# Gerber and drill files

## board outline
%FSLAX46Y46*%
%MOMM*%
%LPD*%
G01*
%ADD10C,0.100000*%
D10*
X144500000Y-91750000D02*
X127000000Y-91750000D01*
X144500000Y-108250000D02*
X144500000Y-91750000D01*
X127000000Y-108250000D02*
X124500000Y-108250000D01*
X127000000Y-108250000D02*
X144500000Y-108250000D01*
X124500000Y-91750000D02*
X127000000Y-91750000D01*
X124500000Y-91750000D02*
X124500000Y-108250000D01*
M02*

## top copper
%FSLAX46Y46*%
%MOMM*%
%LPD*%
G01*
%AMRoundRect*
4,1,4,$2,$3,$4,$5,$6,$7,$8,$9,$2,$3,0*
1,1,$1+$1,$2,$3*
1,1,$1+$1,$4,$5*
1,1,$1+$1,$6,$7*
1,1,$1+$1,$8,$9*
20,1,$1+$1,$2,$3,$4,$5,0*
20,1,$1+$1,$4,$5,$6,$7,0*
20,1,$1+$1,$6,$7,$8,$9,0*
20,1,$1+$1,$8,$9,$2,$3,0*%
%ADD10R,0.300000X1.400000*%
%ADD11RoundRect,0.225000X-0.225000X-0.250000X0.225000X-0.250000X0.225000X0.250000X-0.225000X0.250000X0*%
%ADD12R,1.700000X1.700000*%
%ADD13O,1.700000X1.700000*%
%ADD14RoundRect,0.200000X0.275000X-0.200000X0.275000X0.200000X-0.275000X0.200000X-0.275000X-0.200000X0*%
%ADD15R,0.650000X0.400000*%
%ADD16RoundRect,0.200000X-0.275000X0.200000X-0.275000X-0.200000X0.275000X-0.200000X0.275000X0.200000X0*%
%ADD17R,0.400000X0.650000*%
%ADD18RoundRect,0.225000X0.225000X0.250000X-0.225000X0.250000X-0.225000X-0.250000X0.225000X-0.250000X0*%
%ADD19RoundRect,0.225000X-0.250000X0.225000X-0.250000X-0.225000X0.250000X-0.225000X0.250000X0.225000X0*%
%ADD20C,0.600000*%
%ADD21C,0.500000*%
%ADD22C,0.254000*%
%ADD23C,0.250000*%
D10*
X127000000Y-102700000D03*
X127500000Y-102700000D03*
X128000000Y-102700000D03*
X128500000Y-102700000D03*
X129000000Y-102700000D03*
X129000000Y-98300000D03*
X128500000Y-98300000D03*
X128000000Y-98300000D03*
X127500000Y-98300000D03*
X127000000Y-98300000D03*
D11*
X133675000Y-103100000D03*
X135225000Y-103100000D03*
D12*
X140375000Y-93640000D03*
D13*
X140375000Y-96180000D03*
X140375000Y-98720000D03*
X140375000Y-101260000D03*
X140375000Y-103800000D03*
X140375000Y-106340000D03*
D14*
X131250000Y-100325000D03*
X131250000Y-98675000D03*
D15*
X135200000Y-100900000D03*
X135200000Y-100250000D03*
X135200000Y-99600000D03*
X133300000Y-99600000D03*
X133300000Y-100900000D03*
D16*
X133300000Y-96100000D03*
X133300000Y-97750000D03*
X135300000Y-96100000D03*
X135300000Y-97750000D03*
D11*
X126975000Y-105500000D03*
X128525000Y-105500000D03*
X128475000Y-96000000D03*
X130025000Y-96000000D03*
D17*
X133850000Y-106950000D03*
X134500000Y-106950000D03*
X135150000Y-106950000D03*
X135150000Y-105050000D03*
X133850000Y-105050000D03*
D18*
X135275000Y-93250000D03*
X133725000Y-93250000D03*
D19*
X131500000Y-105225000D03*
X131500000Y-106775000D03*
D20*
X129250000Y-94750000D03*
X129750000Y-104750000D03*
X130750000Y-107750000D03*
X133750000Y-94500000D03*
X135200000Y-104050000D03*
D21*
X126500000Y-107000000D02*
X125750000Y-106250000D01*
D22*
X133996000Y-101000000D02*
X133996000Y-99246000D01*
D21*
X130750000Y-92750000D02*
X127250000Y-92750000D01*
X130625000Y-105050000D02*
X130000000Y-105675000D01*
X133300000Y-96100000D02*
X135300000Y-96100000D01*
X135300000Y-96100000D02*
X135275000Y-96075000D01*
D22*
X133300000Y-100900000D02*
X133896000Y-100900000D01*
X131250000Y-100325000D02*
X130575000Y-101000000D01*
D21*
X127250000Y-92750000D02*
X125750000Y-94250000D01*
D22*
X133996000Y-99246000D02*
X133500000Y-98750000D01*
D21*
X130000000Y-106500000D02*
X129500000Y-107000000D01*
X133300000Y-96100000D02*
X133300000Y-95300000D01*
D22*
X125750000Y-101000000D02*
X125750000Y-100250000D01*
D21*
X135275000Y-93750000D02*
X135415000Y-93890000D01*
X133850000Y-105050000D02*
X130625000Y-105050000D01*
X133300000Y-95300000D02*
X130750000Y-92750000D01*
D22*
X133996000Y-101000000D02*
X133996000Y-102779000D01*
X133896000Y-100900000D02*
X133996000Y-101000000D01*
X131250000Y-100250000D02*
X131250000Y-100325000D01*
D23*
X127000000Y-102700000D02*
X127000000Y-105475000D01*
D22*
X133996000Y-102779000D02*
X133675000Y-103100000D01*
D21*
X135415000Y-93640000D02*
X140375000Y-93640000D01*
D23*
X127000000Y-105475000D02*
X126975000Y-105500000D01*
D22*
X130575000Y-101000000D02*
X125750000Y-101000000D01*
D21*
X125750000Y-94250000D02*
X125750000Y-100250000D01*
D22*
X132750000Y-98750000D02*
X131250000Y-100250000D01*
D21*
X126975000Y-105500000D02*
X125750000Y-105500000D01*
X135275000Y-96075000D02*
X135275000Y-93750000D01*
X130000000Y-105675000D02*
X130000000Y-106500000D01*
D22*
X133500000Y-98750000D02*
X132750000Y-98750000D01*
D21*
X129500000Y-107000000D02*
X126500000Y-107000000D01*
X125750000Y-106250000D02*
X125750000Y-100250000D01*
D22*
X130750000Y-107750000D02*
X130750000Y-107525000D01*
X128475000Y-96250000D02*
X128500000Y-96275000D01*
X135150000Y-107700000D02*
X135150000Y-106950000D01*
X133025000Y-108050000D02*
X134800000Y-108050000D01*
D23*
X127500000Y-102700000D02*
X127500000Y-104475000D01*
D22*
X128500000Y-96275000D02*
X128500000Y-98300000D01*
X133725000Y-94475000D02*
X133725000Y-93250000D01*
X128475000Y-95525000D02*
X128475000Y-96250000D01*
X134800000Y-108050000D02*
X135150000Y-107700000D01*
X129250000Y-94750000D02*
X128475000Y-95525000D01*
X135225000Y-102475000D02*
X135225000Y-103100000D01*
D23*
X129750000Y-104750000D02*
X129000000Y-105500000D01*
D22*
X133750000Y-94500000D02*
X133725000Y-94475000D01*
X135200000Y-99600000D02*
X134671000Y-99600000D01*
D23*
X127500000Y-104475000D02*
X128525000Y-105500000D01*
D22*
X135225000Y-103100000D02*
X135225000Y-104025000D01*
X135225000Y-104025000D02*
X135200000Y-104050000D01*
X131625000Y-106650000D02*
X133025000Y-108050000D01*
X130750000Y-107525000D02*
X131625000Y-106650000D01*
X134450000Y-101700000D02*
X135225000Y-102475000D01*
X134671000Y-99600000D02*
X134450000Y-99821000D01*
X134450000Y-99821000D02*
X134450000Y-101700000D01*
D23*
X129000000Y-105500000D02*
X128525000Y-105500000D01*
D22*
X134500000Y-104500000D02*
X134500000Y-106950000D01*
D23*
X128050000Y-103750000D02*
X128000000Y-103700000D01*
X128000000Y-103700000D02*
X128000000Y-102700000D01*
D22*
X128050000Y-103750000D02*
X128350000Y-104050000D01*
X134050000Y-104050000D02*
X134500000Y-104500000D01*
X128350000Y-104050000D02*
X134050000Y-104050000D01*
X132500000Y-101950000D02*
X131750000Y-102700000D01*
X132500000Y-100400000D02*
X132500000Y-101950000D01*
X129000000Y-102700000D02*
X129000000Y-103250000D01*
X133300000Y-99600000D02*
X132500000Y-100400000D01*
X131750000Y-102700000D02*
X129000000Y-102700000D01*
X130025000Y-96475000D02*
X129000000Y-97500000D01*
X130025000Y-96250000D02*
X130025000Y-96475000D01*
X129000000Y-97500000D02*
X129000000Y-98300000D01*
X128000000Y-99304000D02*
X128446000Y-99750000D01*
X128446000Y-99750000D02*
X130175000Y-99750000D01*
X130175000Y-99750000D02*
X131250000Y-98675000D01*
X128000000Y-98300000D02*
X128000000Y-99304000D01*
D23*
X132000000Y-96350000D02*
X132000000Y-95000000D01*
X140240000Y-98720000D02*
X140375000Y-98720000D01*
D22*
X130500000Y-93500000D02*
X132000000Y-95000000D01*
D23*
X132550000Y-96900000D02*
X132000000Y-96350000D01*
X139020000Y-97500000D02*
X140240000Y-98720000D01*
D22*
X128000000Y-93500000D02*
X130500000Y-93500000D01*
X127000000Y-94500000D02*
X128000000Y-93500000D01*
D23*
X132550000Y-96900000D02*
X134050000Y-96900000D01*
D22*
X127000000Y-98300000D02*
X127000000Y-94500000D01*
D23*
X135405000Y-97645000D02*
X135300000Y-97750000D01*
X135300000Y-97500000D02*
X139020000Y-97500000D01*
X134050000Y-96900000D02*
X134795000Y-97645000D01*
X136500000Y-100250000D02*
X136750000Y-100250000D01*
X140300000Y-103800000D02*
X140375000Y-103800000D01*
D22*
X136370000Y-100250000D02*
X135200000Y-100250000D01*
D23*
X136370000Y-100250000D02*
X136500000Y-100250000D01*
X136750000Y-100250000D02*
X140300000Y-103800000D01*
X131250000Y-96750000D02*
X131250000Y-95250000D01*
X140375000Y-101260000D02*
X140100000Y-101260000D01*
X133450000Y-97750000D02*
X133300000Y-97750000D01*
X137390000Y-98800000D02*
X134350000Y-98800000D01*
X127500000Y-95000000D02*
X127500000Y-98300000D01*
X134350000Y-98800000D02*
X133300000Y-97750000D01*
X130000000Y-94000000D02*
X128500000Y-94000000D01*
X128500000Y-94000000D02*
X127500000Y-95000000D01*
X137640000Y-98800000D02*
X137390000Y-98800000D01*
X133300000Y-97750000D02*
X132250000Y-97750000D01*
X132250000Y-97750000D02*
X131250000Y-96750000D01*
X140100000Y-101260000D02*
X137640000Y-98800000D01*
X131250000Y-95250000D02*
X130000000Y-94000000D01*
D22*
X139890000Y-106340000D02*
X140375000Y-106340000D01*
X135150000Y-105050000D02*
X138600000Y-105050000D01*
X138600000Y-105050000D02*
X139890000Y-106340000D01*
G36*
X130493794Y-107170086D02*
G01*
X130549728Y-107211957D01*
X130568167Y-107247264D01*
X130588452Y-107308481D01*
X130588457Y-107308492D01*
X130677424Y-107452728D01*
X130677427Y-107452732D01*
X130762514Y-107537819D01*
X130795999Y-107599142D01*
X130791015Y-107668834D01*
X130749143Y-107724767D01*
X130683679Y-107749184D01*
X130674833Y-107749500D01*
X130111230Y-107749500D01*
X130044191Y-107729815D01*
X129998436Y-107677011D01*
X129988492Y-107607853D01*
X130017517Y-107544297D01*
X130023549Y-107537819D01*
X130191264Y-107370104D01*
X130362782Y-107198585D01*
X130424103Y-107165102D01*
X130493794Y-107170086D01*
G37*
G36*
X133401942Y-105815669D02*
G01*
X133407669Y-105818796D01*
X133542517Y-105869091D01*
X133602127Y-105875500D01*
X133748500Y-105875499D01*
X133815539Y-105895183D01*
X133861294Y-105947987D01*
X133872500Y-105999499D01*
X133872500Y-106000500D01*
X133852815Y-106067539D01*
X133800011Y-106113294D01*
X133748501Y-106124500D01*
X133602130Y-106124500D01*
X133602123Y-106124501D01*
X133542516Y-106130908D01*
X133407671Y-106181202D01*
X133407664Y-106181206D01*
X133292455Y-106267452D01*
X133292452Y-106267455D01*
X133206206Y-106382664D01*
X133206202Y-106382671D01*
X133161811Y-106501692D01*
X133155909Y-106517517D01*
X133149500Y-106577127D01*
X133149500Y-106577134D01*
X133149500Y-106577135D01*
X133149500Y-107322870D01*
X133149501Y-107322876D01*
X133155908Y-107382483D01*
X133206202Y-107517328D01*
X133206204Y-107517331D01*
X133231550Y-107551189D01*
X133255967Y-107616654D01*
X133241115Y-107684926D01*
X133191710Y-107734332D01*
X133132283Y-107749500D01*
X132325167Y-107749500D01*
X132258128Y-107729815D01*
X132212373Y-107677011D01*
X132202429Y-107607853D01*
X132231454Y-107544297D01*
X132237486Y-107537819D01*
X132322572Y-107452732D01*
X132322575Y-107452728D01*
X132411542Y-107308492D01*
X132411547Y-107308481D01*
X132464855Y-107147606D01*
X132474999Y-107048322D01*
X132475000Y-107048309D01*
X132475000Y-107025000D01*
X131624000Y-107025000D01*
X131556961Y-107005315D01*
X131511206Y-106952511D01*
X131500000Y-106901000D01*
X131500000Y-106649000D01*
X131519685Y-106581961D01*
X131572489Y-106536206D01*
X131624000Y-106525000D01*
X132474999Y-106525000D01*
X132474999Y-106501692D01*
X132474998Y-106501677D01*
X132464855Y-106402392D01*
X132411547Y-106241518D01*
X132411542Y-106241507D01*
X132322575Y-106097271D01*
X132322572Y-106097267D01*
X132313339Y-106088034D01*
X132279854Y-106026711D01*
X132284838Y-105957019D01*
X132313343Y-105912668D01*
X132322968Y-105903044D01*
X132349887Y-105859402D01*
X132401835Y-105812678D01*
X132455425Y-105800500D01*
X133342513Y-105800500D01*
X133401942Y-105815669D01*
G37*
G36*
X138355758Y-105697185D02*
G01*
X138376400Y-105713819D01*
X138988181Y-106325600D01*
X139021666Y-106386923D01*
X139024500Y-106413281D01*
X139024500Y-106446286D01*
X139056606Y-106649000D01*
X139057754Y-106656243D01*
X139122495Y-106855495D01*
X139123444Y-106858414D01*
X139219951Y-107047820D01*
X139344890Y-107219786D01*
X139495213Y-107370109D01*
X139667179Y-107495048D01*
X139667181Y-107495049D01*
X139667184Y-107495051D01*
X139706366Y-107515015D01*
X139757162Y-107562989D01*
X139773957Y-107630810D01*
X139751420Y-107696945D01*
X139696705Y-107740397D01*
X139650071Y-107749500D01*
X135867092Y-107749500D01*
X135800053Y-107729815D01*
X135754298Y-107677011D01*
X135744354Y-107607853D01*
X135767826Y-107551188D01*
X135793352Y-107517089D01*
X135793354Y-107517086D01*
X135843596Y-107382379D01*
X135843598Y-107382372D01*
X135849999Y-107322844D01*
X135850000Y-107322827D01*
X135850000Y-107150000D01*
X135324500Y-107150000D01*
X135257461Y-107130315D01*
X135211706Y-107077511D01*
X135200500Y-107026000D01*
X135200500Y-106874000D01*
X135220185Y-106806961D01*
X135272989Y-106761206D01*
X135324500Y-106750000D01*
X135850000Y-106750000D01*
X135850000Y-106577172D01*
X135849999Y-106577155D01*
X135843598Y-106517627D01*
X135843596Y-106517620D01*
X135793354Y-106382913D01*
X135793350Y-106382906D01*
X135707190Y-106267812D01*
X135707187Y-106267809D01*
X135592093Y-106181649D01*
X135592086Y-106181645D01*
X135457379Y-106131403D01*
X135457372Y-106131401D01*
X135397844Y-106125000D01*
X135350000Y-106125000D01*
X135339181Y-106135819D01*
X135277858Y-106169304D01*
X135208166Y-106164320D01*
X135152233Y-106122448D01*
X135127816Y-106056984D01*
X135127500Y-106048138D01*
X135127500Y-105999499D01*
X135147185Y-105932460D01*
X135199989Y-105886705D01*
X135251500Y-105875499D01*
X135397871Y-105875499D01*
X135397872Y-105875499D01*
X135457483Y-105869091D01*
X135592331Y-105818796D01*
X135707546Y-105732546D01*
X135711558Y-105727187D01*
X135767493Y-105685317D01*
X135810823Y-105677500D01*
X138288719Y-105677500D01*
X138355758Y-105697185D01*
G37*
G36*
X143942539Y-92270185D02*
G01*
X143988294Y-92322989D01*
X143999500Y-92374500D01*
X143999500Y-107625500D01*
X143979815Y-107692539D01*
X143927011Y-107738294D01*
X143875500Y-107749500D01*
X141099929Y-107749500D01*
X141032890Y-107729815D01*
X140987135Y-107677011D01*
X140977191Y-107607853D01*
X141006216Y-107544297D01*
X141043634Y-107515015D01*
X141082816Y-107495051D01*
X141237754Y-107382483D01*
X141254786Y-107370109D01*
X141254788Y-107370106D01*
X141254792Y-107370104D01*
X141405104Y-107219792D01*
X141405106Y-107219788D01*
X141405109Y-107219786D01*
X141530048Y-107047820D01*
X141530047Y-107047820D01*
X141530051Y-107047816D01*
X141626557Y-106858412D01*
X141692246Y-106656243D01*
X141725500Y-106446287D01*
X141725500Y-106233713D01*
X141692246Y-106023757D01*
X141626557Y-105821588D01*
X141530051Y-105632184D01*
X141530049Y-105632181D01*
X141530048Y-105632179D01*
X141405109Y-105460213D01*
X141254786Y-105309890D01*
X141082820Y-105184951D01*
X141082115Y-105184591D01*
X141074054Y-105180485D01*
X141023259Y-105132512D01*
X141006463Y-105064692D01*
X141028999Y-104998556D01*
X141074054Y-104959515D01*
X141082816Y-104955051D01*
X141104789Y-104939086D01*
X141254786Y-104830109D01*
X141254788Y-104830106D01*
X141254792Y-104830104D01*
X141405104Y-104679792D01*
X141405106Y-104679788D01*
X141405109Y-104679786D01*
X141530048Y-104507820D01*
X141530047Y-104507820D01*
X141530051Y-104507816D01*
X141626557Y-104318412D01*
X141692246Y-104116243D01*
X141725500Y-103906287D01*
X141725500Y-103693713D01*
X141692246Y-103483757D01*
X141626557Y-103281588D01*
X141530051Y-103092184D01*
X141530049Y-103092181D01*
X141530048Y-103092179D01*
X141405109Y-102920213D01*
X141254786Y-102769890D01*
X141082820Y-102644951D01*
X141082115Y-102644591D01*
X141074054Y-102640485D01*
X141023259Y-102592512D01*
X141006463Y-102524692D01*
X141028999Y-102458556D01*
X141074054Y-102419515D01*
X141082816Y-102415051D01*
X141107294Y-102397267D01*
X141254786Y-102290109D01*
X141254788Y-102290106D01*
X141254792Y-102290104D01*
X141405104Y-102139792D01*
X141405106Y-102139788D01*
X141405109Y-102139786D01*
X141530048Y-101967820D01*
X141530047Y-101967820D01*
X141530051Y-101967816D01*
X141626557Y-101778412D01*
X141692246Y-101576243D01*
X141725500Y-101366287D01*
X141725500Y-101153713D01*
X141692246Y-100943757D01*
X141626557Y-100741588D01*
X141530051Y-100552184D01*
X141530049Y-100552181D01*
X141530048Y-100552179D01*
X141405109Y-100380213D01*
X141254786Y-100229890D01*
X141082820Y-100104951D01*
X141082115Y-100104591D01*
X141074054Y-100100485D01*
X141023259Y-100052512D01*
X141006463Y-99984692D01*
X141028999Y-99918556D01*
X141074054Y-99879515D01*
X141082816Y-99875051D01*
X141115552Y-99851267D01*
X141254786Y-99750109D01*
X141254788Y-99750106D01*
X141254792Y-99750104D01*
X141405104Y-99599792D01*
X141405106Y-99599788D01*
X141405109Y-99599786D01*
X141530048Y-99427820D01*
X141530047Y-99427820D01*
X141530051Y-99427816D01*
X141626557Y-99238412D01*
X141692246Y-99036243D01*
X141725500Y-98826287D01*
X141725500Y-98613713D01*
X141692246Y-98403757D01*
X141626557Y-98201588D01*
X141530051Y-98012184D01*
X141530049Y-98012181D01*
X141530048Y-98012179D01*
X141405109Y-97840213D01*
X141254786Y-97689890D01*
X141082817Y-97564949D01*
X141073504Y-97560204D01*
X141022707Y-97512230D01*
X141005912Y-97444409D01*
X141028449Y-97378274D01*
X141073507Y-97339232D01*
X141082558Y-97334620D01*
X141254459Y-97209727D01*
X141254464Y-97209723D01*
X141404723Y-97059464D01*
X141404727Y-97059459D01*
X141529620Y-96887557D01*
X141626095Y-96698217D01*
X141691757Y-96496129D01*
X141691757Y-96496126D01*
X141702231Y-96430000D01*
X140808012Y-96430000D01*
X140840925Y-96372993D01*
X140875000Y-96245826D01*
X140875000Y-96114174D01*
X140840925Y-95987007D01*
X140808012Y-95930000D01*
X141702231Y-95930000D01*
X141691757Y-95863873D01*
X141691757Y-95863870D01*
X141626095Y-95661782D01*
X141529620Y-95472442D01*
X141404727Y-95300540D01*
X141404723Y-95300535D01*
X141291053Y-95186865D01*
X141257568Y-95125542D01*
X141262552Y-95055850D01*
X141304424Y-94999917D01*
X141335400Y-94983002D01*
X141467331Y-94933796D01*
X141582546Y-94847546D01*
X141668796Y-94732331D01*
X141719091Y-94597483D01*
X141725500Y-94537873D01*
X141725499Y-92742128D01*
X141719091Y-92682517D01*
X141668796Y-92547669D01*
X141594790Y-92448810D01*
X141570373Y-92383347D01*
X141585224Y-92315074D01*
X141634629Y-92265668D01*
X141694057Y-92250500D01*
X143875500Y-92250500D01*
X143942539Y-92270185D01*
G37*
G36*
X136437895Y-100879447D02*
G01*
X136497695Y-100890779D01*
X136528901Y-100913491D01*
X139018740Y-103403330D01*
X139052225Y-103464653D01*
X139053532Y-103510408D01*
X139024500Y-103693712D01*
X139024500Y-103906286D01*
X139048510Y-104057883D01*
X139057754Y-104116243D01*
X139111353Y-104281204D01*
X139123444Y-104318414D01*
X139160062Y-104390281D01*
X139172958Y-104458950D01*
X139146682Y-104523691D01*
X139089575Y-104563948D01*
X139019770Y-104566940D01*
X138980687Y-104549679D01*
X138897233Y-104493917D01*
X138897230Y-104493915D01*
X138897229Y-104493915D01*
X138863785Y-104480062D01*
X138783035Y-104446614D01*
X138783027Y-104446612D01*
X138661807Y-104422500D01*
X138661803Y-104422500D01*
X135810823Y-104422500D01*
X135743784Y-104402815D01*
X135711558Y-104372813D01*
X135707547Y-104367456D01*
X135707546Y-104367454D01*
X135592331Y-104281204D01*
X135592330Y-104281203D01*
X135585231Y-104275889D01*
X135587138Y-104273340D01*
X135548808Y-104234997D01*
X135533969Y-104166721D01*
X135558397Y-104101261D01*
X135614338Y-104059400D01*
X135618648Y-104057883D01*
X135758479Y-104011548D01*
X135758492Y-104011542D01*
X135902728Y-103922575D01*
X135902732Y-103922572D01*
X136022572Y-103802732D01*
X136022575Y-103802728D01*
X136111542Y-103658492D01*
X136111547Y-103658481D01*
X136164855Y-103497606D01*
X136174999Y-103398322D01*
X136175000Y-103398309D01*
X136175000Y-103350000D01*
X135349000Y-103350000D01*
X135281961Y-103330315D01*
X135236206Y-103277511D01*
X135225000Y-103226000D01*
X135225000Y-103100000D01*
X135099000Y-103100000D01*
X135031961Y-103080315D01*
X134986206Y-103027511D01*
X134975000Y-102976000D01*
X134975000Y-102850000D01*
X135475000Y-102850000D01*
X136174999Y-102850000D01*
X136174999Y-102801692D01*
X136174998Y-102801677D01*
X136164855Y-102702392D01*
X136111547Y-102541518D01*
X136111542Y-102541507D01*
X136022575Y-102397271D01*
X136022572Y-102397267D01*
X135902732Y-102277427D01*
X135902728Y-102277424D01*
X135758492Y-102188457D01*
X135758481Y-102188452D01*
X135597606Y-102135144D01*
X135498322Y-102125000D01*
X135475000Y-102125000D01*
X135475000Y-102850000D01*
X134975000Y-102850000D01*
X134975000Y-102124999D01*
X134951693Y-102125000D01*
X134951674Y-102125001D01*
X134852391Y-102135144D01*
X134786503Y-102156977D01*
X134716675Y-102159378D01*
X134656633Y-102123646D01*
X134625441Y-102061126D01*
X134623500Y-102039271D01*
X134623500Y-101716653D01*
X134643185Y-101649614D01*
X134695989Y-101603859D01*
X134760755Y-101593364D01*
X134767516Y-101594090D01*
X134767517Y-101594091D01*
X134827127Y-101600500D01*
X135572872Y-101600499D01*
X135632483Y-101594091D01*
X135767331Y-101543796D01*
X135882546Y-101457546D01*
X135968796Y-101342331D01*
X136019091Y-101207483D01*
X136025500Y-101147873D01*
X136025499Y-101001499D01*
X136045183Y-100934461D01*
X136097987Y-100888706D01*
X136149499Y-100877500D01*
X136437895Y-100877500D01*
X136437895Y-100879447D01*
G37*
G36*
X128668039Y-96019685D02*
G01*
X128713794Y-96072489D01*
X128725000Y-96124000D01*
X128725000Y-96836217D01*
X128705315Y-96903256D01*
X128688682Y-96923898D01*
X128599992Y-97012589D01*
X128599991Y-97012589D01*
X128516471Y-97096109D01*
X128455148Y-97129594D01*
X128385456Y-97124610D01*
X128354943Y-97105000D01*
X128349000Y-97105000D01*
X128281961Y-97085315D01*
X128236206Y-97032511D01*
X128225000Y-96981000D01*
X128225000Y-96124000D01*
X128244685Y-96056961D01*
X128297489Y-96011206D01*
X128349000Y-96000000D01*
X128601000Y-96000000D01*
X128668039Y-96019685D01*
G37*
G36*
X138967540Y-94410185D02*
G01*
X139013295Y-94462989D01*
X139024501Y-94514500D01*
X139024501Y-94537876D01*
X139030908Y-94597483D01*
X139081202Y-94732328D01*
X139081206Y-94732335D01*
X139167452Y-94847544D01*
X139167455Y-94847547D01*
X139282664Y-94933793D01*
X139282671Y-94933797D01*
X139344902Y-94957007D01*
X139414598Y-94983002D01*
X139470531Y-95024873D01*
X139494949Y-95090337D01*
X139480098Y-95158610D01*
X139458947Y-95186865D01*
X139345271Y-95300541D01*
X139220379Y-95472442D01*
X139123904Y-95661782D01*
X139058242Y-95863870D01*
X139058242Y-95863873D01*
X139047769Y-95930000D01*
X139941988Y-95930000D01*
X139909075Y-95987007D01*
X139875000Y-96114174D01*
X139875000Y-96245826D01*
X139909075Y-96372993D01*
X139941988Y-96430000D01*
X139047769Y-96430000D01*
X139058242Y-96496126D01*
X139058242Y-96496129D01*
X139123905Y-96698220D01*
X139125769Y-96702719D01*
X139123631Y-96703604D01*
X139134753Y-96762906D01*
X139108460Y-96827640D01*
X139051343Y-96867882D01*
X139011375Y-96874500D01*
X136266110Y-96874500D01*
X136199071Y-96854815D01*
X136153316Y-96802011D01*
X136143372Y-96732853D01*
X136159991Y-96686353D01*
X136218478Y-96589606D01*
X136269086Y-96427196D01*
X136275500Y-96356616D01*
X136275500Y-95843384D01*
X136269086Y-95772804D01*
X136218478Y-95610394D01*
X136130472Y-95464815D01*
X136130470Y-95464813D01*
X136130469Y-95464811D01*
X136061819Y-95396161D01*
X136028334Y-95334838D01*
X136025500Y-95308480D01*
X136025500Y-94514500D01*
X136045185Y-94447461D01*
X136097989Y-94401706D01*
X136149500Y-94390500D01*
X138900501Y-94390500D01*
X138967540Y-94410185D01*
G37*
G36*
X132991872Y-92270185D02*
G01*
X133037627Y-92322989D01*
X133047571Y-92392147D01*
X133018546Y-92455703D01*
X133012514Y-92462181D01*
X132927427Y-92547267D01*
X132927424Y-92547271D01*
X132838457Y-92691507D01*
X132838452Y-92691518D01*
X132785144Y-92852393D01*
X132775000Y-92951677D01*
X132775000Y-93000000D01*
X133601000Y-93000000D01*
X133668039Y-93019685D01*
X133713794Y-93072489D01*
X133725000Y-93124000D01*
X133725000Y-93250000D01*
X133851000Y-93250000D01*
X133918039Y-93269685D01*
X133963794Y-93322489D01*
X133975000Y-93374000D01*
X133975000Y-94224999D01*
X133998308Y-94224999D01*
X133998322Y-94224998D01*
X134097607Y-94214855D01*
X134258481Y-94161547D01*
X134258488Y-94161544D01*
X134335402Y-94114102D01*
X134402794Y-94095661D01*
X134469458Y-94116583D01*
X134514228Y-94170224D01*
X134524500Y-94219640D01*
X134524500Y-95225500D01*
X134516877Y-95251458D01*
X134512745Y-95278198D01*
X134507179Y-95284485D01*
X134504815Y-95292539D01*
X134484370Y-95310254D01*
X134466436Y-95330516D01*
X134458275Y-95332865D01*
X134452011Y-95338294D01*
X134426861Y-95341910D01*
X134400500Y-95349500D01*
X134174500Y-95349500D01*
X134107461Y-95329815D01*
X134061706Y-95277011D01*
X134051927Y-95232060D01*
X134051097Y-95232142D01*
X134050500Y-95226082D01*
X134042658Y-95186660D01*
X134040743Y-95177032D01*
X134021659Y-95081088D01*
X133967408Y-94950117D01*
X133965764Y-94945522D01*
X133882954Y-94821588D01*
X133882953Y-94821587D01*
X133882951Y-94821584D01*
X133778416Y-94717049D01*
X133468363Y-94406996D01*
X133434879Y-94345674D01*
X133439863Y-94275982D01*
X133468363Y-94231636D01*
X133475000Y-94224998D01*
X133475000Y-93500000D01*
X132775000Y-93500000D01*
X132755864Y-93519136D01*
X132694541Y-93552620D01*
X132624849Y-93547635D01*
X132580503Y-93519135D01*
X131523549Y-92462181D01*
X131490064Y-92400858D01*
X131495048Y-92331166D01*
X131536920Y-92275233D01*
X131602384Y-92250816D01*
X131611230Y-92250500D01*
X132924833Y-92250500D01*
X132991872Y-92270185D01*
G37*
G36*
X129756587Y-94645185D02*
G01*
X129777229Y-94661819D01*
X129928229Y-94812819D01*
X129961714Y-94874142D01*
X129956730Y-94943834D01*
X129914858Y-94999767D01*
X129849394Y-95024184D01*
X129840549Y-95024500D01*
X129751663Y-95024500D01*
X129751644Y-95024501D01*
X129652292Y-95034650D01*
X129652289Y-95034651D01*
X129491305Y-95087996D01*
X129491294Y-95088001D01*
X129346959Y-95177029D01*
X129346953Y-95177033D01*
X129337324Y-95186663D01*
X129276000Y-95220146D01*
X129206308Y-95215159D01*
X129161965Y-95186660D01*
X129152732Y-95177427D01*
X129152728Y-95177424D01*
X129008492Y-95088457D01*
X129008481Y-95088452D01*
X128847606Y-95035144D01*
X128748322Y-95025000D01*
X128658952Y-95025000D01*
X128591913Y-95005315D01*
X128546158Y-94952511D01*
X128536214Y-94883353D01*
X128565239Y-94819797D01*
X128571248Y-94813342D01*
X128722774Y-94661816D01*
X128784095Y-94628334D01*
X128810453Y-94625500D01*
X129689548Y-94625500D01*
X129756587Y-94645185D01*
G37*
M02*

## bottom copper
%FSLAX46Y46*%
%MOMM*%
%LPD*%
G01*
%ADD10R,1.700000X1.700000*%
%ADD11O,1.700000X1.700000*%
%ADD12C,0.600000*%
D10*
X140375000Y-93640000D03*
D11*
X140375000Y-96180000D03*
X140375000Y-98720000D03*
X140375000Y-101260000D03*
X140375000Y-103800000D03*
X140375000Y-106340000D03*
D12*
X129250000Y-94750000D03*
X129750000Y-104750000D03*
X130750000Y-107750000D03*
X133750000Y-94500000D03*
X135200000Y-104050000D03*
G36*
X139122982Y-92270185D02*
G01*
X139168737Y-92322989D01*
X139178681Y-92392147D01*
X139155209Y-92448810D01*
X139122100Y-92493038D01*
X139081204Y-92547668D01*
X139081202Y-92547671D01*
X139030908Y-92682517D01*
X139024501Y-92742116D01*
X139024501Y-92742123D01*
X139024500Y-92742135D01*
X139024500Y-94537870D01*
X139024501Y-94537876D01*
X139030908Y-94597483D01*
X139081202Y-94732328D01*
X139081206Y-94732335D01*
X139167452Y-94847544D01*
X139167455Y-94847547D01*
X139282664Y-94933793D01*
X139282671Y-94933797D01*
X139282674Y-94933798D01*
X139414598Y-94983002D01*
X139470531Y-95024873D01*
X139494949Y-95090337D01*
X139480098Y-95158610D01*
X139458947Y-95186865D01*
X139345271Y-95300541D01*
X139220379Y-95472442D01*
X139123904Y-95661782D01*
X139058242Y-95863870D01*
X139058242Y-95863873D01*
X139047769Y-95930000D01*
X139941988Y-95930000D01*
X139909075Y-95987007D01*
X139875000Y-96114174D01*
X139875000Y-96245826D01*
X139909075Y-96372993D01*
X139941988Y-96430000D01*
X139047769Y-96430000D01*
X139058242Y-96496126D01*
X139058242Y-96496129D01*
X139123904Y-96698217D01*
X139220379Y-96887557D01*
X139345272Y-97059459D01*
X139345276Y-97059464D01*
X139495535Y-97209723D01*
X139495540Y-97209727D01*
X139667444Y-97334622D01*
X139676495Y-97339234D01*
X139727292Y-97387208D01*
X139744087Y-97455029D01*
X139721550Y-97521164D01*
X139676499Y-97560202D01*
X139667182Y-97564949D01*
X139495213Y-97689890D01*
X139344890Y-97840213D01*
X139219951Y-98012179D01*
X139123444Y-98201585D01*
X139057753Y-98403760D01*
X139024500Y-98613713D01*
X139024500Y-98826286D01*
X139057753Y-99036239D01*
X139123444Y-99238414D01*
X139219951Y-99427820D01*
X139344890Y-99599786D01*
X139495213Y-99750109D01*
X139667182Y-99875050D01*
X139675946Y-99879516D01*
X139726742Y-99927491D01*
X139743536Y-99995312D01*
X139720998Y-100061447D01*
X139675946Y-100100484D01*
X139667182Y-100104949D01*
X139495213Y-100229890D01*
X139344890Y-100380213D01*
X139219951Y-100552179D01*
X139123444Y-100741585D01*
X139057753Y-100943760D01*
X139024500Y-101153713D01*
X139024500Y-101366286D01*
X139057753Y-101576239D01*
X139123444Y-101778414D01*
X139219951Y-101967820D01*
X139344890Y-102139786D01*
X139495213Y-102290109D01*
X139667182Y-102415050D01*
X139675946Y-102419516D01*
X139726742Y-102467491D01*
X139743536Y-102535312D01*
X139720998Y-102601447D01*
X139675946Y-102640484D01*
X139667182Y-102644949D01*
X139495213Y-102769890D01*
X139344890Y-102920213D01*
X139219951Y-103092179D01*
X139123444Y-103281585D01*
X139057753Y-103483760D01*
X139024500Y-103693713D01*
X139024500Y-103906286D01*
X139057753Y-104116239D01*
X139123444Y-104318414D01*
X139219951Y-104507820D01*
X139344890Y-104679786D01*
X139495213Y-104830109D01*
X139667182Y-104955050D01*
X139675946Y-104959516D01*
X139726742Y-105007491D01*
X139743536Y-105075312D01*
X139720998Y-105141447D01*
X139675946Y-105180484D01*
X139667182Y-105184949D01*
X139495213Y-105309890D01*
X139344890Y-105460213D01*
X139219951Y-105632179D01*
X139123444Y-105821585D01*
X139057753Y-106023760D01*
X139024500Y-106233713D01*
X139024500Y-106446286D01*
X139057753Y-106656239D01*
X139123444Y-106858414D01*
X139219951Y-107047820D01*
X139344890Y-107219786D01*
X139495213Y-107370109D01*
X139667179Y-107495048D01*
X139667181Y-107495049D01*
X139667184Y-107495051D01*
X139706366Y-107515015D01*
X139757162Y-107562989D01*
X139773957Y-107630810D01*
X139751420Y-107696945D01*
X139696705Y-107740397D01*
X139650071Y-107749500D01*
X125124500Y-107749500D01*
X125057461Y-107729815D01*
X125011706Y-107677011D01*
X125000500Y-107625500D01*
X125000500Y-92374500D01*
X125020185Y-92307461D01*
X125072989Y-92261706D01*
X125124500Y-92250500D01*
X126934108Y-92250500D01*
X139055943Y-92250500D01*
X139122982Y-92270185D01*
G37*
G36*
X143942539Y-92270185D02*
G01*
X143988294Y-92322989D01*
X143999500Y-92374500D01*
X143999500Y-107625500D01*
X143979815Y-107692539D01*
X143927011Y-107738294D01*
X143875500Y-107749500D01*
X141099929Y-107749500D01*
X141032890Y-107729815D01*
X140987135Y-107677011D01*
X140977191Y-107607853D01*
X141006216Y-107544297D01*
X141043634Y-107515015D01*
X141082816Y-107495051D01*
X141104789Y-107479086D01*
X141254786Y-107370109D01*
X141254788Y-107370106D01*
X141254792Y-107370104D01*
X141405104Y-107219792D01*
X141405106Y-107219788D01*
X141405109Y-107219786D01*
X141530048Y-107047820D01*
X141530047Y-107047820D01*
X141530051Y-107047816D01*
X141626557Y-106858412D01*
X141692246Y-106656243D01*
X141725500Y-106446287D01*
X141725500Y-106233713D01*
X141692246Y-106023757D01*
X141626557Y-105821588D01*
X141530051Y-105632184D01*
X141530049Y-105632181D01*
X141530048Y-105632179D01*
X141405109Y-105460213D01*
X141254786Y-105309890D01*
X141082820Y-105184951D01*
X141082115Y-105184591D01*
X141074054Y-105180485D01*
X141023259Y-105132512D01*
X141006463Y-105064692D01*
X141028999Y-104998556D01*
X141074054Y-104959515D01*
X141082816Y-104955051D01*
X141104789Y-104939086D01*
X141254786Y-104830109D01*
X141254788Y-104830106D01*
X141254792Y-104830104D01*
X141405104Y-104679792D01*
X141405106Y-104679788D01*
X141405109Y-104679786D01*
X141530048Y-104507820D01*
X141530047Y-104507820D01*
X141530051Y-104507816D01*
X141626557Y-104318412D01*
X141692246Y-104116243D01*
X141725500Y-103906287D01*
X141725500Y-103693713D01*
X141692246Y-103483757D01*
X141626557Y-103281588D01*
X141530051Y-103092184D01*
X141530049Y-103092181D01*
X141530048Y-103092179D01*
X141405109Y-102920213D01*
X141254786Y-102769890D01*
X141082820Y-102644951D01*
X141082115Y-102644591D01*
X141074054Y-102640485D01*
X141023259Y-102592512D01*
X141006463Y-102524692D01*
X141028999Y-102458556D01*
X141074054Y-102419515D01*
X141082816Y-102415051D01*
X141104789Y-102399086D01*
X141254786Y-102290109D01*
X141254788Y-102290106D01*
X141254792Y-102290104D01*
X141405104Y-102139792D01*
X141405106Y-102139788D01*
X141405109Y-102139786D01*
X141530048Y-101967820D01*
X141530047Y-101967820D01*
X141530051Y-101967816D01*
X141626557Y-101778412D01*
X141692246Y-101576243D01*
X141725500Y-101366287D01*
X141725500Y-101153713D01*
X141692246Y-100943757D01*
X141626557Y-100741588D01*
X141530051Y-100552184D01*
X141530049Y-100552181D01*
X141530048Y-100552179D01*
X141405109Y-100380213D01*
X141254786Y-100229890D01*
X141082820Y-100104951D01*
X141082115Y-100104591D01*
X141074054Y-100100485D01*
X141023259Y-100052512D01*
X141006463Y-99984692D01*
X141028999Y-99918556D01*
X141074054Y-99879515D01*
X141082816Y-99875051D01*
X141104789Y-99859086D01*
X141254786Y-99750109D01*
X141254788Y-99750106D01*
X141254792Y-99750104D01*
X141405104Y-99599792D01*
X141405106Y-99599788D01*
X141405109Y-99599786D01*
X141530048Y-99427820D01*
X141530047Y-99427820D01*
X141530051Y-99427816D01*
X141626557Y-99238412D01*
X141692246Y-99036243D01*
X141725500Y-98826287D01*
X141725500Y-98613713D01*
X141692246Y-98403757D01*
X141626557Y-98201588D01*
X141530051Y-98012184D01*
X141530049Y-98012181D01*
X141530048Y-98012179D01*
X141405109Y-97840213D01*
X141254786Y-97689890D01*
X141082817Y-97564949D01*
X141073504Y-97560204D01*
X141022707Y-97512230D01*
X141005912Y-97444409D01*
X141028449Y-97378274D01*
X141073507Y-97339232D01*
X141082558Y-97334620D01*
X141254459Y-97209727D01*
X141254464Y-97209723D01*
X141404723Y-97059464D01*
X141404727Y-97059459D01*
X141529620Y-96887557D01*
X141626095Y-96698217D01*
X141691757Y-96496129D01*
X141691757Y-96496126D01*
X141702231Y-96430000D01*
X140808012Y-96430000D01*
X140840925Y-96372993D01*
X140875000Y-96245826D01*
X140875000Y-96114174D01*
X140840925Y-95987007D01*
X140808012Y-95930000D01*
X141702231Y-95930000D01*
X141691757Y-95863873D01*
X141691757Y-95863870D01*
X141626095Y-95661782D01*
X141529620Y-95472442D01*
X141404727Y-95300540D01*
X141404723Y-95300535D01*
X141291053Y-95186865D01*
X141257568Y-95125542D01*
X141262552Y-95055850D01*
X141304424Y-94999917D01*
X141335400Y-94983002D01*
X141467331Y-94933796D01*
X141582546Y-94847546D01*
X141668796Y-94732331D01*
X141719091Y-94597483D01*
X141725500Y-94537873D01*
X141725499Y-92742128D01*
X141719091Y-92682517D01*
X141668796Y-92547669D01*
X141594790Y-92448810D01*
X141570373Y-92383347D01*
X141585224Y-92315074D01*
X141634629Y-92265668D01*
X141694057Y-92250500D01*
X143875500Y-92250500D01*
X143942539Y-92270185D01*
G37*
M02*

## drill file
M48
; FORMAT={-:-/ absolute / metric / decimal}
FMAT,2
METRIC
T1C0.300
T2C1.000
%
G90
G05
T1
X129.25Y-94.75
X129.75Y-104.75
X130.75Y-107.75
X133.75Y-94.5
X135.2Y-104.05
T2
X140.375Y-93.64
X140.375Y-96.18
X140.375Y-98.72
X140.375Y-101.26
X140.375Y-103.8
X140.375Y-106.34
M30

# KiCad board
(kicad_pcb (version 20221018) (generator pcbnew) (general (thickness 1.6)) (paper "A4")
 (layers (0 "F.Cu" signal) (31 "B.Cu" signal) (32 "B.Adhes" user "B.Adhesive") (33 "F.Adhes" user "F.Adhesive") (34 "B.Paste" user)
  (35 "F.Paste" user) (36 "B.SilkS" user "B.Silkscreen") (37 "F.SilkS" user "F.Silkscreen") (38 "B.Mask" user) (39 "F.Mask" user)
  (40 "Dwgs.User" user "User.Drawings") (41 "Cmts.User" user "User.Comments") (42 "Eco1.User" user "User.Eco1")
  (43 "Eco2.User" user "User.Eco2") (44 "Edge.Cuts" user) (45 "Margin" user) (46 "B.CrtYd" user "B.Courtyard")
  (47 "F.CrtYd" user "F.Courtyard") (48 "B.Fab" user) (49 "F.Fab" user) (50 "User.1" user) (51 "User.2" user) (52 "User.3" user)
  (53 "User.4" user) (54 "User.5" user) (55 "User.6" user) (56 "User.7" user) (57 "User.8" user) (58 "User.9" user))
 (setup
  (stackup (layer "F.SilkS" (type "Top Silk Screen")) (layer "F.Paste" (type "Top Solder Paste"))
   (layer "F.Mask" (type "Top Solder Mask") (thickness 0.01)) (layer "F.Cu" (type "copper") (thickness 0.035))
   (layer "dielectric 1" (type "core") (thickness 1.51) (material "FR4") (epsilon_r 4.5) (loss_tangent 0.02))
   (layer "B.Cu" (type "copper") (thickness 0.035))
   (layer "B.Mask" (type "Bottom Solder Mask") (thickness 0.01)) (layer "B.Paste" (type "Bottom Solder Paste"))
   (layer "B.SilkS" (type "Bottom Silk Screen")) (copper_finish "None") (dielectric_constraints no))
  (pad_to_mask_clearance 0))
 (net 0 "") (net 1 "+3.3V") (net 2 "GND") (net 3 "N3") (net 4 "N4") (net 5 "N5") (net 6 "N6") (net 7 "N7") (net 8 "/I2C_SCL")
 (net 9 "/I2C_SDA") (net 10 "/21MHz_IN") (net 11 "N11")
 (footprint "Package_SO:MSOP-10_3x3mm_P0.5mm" (layer "F.Cu") (at 128 100.5 90)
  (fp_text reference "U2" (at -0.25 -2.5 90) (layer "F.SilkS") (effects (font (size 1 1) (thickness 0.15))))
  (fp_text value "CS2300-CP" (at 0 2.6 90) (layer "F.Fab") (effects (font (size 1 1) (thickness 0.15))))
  (pad "1" smd rect (at -2.2 -1 90) (size 1.4 0.3) (layers "F.Cu" "F.Paste" "F.Mask") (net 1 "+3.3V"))
  (pad "2" smd rect (at -2.2 -0.5 90) (size 1.4 0.3) (layers "F.Cu" "F.Paste" "F.Mask") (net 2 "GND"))
  (pad "3" smd rect (at -2.2 0 90) (size 1.4 0.3) (layers "F.Cu" "F.Paste" "F.Mask") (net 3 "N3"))
  (pad "4" smd rect (at -2.2 0.5 90) (size 1.4 0.3) (layers "F.Cu" "F.Paste" "F.Mask") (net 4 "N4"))
  (pad "5" smd rect (at -2.2 1 90) (size 1.4 0.3) (layers "F.Cu" "F.Paste" "F.Mask") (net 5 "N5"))
  (pad "6" smd rect (at 2.2 1 90) (size 1.4 0.3) (layers "F.Cu" "F.Paste" "F.Mask") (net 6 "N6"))
  (pad "7" smd rect (at 2.2 0.5 90) (size 1.4 0.3) (layers "F.Cu" "F.Paste" "F.Mask") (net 2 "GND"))
  (pad "8" smd rect (at 2.2 0 90) (size 1.4 0.3) (layers "F.Cu" "F.Paste" "F.Mask") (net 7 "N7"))
  (pad "9" smd rect (at 2.2 -0.5 90) (size 1.4 0.3) (layers "F.Cu" "F.Paste" "F.Mask") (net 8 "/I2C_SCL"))
  (pad "10" smd rect (at 2.2 -1 90) (size 1.4 0.3) (layers "F.Cu" "F.Paste" "F.Mask") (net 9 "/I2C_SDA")))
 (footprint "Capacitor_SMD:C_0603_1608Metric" (layer "F.Cu") (at 134.45 103.1)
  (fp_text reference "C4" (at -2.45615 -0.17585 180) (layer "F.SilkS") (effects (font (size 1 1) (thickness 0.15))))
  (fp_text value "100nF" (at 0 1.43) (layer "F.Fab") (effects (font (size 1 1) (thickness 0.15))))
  (pad "1" smd roundrect (at -0.775 0) (size 0.9 0.95) (layers "F.Cu" "F.Paste" "F.Mask") (roundrect_rratio 0.25) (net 1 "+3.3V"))
  (pad "2" smd roundrect (at 0.775 0) (size 0.9 0.95) (layers "F.Cu" "F.Paste" "F.Mask") (roundrect_rratio 0.25) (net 2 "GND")))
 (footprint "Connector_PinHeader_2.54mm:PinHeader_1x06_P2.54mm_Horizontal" (layer "F.Cu") (at 140.375 93.64)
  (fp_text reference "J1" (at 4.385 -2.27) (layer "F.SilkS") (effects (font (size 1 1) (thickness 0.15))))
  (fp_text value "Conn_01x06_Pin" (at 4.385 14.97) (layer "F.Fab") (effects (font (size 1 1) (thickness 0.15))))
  (pad "1" thru_hole rect (at 0 0) (size 1.7 1.7) (drill 1) (layers "*.Cu" "*.Mask") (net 1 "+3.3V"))
  (pad "2" thru_hole oval (at 0 2.54) (size 1.7 1.7) (drill 1) (layers "*.Cu" "*.Mask") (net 2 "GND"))
  (pad "3" thru_hole oval (at 0 5.08) (size 1.7 1.7) (drill 1) (layers "*.Cu" "*.Mask") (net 9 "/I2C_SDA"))
  (pad "4" thru_hole oval (at 0 7.62) (size 1.7 1.7) (drill 1) (layers "*.Cu" "*.Mask") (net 8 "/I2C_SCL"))
  (pad "5" thru_hole oval (at 0 10.16) (size 1.7 1.7) (drill 1) (layers "*.Cu" "*.Mask") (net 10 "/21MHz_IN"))
  (pad "6" thru_hole oval (at 0 12.7) (size 1.7 1.7) (drill 1) (layers "*.Cu" "*.Mask") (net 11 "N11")))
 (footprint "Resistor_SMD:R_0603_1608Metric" (layer "F.Cu") (at 131.25 99.5 90)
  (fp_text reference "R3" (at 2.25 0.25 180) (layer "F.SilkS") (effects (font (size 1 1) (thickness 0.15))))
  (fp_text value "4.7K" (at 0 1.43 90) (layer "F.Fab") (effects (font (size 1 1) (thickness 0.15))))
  (pad "1" smd roundrect (at -0.825 0 90) (size 0.8 0.95) (layers "F.Cu" "F.Paste" "F.Mask") (roundrect_rratio 0.25) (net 1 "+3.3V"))
  (pad "2" smd roundrect (at 0.825 0 90) (size 0.8 0.95) (layers "F.Cu" "F.Paste" "F.Mask") (roundrect_rratio 0.25) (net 7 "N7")))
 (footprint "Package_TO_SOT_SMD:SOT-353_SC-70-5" (layer "F.Cu") (at 134.25 100.25 180)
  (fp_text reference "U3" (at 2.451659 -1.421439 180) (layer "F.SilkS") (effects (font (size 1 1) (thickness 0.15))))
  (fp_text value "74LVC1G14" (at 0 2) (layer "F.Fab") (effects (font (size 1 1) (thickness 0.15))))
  (pad "1" smd rect (at -0.95 -0.65 180) (size 0.65 0.4) (layers "F.Cu" "F.Paste" "F.Mask"))
  (pad "2" smd rect (at -0.95 0 180) (size 0.65 0.4) (layers "F.Cu" "F.Paste" "F.Mask") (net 10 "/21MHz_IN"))
  (pad "3" smd rect (at -0.95 0.65 180) (size 0.65 0.4) (layers "F.Cu" "F.Paste" "F.Mask") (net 2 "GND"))
  (pad "4" smd rect (at 0.95 0.65 180) (size 0.65 0.4) (layers "F.Cu" "F.Paste" "F.Mask") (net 5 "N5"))
  (pad "5" smd rect (at 0.95 -0.65 180) (size 0.65 0.4) (layers "F.Cu" "F.Paste" "F.Mask") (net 1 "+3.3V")))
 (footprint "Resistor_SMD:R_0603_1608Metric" (layer "F.Cu") (at 133.3 96.925 -90)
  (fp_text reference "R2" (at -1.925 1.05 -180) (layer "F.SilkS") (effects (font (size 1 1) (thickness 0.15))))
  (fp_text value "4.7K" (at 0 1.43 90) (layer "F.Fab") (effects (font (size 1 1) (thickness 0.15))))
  (pad "1" smd roundrect (at -0.825 0 270) (size 0.8 0.95) (layers "F.Cu" "F.Paste" "F.Mask") (roundrect_rratio 0.25) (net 1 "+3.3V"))
  (pad "2" smd roundrect (at 0.825 0 270) (size 0.8 0.95) (layers "F.Cu" "F.Paste" "F.Mask") (roundrect_rratio 0.25) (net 8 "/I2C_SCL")))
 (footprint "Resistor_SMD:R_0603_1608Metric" (layer "F.Cu") (at 135.3 96.925 -90)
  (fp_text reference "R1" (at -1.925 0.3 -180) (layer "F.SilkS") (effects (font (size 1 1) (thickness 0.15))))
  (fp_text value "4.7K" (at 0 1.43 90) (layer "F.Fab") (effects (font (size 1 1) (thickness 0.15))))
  (pad "1" smd roundrect (at -0.825 0 270) (size 0.8 0.95) (layers "F.Cu" "F.Paste" "F.Mask") (roundrect_rratio 0.25) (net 1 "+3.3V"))
  (pad "2" smd roundrect (at 0.825 0 270) (size 0.8 0.95) (layers "F.Cu" "F.Paste" "F.Mask") (roundrect_rratio 0.25) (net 9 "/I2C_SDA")))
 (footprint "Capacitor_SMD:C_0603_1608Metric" (layer "F.Cu") (at 127.75 105.5)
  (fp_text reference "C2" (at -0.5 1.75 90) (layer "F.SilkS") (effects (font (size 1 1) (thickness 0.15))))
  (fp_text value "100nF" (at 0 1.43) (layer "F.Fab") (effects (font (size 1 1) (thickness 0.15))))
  (pad "1" smd roundrect (at -0.775 0) (size 0.9 0.95) (layers "F.Cu" "F.Paste" "F.Mask") (roundrect_rratio 0.25) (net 1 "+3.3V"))
  (pad "2" smd roundrect (at 0.775 0) (size 0.9 0.95) (layers "F.Cu" "F.Paste" "F.Mask") (roundrect_rratio 0.25) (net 2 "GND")))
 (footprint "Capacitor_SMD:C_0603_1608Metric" (layer "F.Cu") (at 129.25 96)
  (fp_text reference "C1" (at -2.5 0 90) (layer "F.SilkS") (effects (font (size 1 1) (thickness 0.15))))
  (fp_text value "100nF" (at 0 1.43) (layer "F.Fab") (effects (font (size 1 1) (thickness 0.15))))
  (pad "1" smd roundrect (at -0.775 0) (size 0.9 0.95) (layers "F.Cu" "F.Paste" "F.Mask") (roundrect_rratio 0.25) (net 2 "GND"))
  (pad "2" smd roundrect (at 0.775 0) (size 0.9 0.95) (layers "F.Cu" "F.Paste" "F.Mask") (roundrect_rratio 0.25) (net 6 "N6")))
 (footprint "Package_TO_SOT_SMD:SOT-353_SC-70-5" (layer "F.Cu") (at 134.5 106 90)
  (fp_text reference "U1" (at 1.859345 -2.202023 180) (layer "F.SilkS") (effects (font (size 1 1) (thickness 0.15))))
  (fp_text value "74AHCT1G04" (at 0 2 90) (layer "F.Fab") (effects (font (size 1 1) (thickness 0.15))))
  (pad "1" smd rect (at -0.95 -0.65 90) (size 0.65 0.4) (layers "F.Cu" "F.Paste" "F.Mask"))
  (pad "2" smd rect (at -0.95 0 90) (size 0.65 0.4) (layers "F.Cu" "F.Paste" "F.Mask") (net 3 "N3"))
  (pad "3" smd rect (at -0.95 0.65 90) (size 0.65 0.4) (layers "F.Cu" "F.Paste" "F.Mask") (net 2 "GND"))
  (pad "4" smd rect (at 0.95 0.65 90) (size 0.65 0.4) (layers "F.Cu" "F.Paste" "F.Mask") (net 11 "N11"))
  (pad "5" smd rect (at 0.95 -0.65 90) (size 0.65 0.4) (layers "F.Cu" "F.Paste" "F.Mask") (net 1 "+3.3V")))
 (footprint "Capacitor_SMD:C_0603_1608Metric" (layer "F.Cu") (at 134.5 93.25 180)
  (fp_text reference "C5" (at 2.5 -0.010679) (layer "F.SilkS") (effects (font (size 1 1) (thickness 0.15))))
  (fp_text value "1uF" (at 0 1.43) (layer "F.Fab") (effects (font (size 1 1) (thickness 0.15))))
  (pad "1" smd roundrect (at -0.775 0 180) (size 0.9 0.95) (layers "F.Cu" "F.Paste" "F.Mask") (roundrect_rratio 0.25) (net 1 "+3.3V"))
  (pad "2" smd roundrect (at 0.775 0 180) (size 0.9 0.95) (layers "F.Cu" "F.Paste" "F.Mask") (roundrect_rratio 0.25) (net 2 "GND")))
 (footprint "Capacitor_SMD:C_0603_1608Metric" (layer "F.Cu") (at 131.5 106 -90)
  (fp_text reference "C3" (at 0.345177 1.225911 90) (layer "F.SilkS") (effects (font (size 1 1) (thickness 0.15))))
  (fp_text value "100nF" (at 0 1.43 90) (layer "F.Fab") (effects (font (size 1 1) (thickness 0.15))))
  (pad "1" smd roundrect (at -0.775 0 270) (size 0.9 0.95) (layers "F.Cu" "F.Paste" "F.Mask") (roundrect_rratio 0.25) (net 1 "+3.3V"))
  (pad "2" smd roundrect (at 0.775 0 270) (size 0.9 0.95) (layers "F.Cu" "F.Paste" "F.Mask") (roundrect_rratio 0.25) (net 2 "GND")))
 (gr_line (start 144.5 91.75) (end 127 91.75) (stroke (width 0.1) (type default)) (layer "Edge.Cuts"))
 (gr_line (start 144.5 108.25) (end 144.5 91.75) (stroke (width 0.1) (type default)) (layer "Edge.Cuts"))
 (gr_line (start 127 108.25) (end 124.5 108.25) (stroke (width 0.1) (type default)) (layer "Edge.Cuts"))
 (gr_line (start 127 108.25) (end 144.5 108.25) (stroke (width 0.1) (type default)) (layer "Edge.Cuts"))
 (gr_line (start 124.5 91.75) (end 127 91.75) (stroke (width 0.1) (type default)) (layer "Edge.Cuts"))
 (gr_line (start 124.5 91.75) (end 124.5 108.25) (stroke (width 0.1) (type default)) (layer "Edge.Cuts"))
 (segment (start 126.5 107) (end 125.75 106.25) (width 0.5) (layer "F.Cu") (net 1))
 (segment (start 133.996 101) (end 133.996 99.246) (width 0.254) (layer "F.Cu") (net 1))
 (segment (start 130.75 92.75) (end 127.25 92.75) (width 0.5) (layer "F.Cu") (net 1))
 (segment (start 130.625 105.05) (end 130 105.675) (width 0.5) (layer "F.Cu") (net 1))
 (segment (start 133.3 96.1) (end 135.3 96.1) (width 0.5) (layer "F.Cu") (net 1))
 (segment (start 135.3 96.1) (end 135.275 96.075) (width 0.5) (layer "F.Cu") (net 1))
 (segment (start 133.3 100.9) (end 133.896 100.9) (width 0.254) (layer "F.Cu") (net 1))
 (segment (start 131.25 100.325) (end 130.575 101) (width 0.254) (layer "F.Cu") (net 1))
 (segment (start 127.25 92.75) (end 125.75 94.25) (width 0.5) (layer "F.Cu") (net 1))
 (segment (start 133.996 99.246) (end 133.5 98.75) (width 0.254) (layer "F.Cu") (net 1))
 (segment (start 130 106.5) (end 129.5 107) (width 0.5) (layer "F.Cu") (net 1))
 (segment (start 133.3 96.1) (end 133.3 95.3) (width 0.5) (layer "F.Cu") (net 1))
 (segment (start 125.75 101) (end 125.75 100.25) (width 0.254) (layer "F.Cu") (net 1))
 (segment (start 135.275 93.75) (end 135.415 93.89) (width 0.5) (layer "F.Cu") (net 1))
 (segment (start 133.85 105.05) (end 130.625 105.05) (width 0.5) (layer "F.Cu") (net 1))
 (segment (start 133.3 95.3) (end 130.75 92.75) (width 0.5) (layer "F.Cu") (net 1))
 (segment (start 133.996 101) (end 133.996 102.779) (width 0.254) (layer "F.Cu") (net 1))
 (segment (start 133.896 100.9) (end 133.996 101) (width 0.254) (layer "F.Cu") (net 1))
 (segment (start 131.25 100.25) (end 131.25 100.325) (width 0.254) (layer "F.Cu") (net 1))
 (segment (start 127 102.7) (end 127 105.475) (width 0.25) (layer "F.Cu") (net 1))
 (segment (start 133.996 102.779) (end 133.675 103.1) (width 0.254) (layer "F.Cu") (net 1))
 (segment (start 135.415 93.64) (end 140.375 93.64) (width 0.5) (layer "F.Cu") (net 1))
 (segment (start 127 105.475) (end 126.975 105.5) (width 0.25) (layer "F.Cu") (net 1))
 (segment (start 130.575 101) (end 125.75 101) (width 0.254) (layer "F.Cu") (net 1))
 (segment (start 125.75 94.25) (end 125.75 100.25) (width 0.5) (layer "F.Cu") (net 1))
 (segment (start 132.75 98.75) (end 131.25 100.25) (width 0.254) (layer "F.Cu") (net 1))
 (segment (start 126.975 105.5) (end 125.75 105.5) (width 0.5) (layer "F.Cu") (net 1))
 (segment (start 135.275 96.075) (end 135.275 93.75) (width 0.5) (layer "F.Cu") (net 1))
 (segment (start 130 105.675) (end 130 106.5) (width 0.5) (layer "F.Cu") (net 1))
 (segment (start 133.5 98.75) (end 132.75 98.75) (width 0.254) (layer "F.Cu") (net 1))
 (segment (start 129.5 107) (end 126.5 107) (width 0.5) (layer "F.Cu") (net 1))
 (segment (start 125.75 106.25) (end 125.75 100.25) (width 0.5) (layer "F.Cu") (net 1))
 (segment (start 130.75 107.75) (end 130.75 107.525) (width 0.254) (layer "F.Cu") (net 2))
 (segment (start 128.475 96.25) (end 128.5 96.275) (width 0.254) (layer "F.Cu") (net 2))
 (segment (start 135.15 107.7) (end 135.15 106.95) (width 0.254) (layer "F.Cu") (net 2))
 (segment (start 133.025 108.05) (end 134.8 108.05) (width 0.254) (layer "F.Cu") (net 2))
 (segment (start 127.5 102.7) (end 127.5 104.475) (width 0.25) (layer "F.Cu") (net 2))
 (segment (start 128.5 96.275) (end 128.5 98.3) (width 0.254) (layer "F.Cu") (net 2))
 (segment (start 133.725 94.475) (end 133.725 93.25) (width 0.254) (layer "F.Cu") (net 2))
 (segment (start 128.475 95.525) (end 128.475 96.25) (width 0.254) (layer "F.Cu") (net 2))
 (segment (start 134.8 108.05) (end 135.15 107.7) (width 0.254) (layer "F.Cu") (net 2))
 (segment (start 129.25 94.75) (end 128.475 95.525) (width 0.254) (layer "F.Cu") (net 2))
 (segment (start 135.225 102.475) (end 135.225 103.1) (width 0.254) (layer "F.Cu") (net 2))
 (segment (start 129.75 104.75) (end 129 105.5) (width 0.25) (layer "F.Cu") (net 2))
 (segment (start 133.75 94.5) (end 133.725 94.475) (width 0.254) (layer "F.Cu") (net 2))
 (segment (start 135.2 99.6) (end 134.671 99.6) (width 0.254) (layer "F.Cu") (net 2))
 (segment (start 127.5 104.475) (end 128.525 105.5) (width 0.25) (layer "F.Cu") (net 2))
 (segment (start 135.225 103.1) (end 135.225 104.025) (width 0.254) (layer "F.Cu") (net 2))
 (segment (start 135.225 104.025) (end 135.2 104.05) (width 0.254) (layer "F.Cu") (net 2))
 (segment (start 131.625 106.65) (end 133.025 108.05) (width 0.254) (layer "F.Cu") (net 2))
 (segment (start 130.75 107.525) (end 131.625 106.65) (width 0.254) (layer "F.Cu") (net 2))
 (segment (start 134.45 101.7) (end 135.225 102.475) (width 0.254) (layer "F.Cu") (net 2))
 (segment (start 134.671 99.6) (end 134.45 99.821) (width 0.254) (layer "F.Cu") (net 2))
 (segment (start 134.45 99.821) (end 134.45 101.7) (width 0.254) (layer "F.Cu") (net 2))
 (segment (start 129 105.5) (end 128.525 105.5) (width 0.25) (layer "F.Cu") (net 2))
 (via (at 129.25 94.75) (size 0.6) (drill 0.3) (layers "F.Cu" "B.Cu") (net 2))
 (via (at 129.75 104.75) (size 0.6) (drill 0.3) (layers "F.Cu" "B.Cu") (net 2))
 (via (at 130.75 107.75) (size 0.6) (drill 0.3) (layers "F.Cu" "B.Cu") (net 2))
 (via (at 133.75 94.5) (size 0.6) (drill 0.3) (layers "F.Cu" "B.Cu") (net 2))
 (via (at 135.2 104.05) (size 0.6) (drill 0.3) (layers "F.Cu" "B.Cu") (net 2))
 (segment (start 134.5 104.5) (end 134.5 106.95) (width 0.254) (layer "F.Cu") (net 3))
 (segment (start 128.05 103.75) (end 128 103.7) (width 0.25) (layer "F.Cu") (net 3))
 (segment (start 128 103.7) (end 128 102.7) (width 0.25) (layer "F.Cu") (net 3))
 (segment (start 128.05 103.75) (end 128.35 104.05) (width 0.254) (layer "F.Cu") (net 3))
 (segment (start 134.05 104.05) (end 134.5 104.5) (width 0.254) (layer "F.Cu") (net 3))
 (segment (start 128.35 104.05) (end 134.05 104.05) (width 0.254) (layer "F.Cu") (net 3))
 (segment (start 132.5 101.95) (end 131.75 102.7) (width 0.254) (layer "F.Cu") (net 5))
 (segment (start 132.5 100.4) (end 132.5 101.95) (width 0.254) (layer "F.Cu") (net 5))
 (segment (start 129 102.7) (end 129 103.25) (width 0.254) (layer "F.Cu") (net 5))
 (segment (start 133.3 99.6) (end 132.5 100.4) (width 0.254) (layer "F.Cu") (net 5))
 (segment (start 131.75 102.7) (end 129 102.7) (width 0.254) (layer "F.Cu") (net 5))
 (segment (start 130.025 96.475) (end 129 97.5) (width 0.254) (layer "F.Cu") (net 6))
 (segment (start 130.025 96.25) (end 130.025 96.475) (width 0.254) (layer "F.Cu") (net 6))
 (segment (start 129 97.5) (end 129 98.3) (width 0.254) (layer "F.Cu") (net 6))
 (segment (start 128 99.304) (end 128.446 99.75) (width 0.254) (layer "F.Cu") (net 7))
 (segment (start 128.446 99.75) (end 130.175 99.75) (width 0.254) (layer "F.Cu") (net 7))
 (segment (start 130.175 99.75) (end 131.25 98.675) (width 0.254) (layer "F.Cu") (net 7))
 (segment (start 128 98.3) (end 128 99.304) (width 0.254) (layer "F.Cu") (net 7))
 (segment (start 132 96.35) (end 132 95) (width 0.25) (layer "F.Cu") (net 9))
 (segment (start 140.24 98.72) (end 140.375 98.72) (width 0.25) (layer "F.Cu") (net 9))
 (segment (start 130.5 93.5) (end 132 95) (width 0.254) (layer "F.Cu") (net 9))
 (segment (start 132.55 96.9) (end 132 96.35) (width 0.25) (layer "F.Cu") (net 9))
 (segment (start 139.02 97.5) (end 140.24 98.72) (width 0.25) (layer "F.Cu") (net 9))
 (segment (start 128 93.5) (end 130.5 93.5) (width 0.254) (layer "F.Cu") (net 9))
 (segment (start 127 94.5) (end 128 93.5) (width 0.254) (layer "F.Cu") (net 9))
 (segment (start 132.55 96.9) (end 134.05 96.9) (width 0.25) (layer "F.Cu") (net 9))
 (segment (start 127 98.3) (end 127 94.5) (width 0.254) (layer "F.Cu") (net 9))
 (segment (start 135.405 97.645) (end 135.3 97.75) (width 0.25) (layer "F.Cu") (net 9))
 (segment (start 135.3 97.5) (end 139.02 97.5) (width 0.25) (layer "F.Cu") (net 9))
 (segment (start 134.05 96.9) (end 134.795 97.645) (width 0.25) (layer "F.Cu") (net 9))
 (segment (start 136.5 100.25) (end 136.75 100.25) (width 0.25) (layer "F.Cu") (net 10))
 (segment (start 140.3 103.8) (end 140.375 103.8) (width 0.25) (layer "F.Cu") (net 10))
 (segment (start 136.37 100.25) (end 135.2 100.25) (width 0.254) (layer "F.Cu") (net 10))
 (segment (start 136.37 100.25) (end 136.5 100.25) (width 0.25) (layer "F.Cu") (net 10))
 (segment (start 136.75 100.25) (end 140.3 103.8) (width 0.25) (layer "F.Cu") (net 10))
 (segment (start 131.25 96.75) (end 131.25 95.25) (width 0.25) (layer "F.Cu") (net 8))
 (segment (start 140.375 101.26) (end 140.1 101.26) (width 0.25) (layer "F.Cu") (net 8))
 (segment (start 133.45 97.75) (end 133.3 97.75) (width 0.25) (layer "F.Cu") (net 8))
 (segment (start 137.39 98.8) (end 134.35 98.8) (width 0.25) (layer "F.Cu") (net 8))
 (segment (start 127.5 95) (end 127.5 98.3) (width 0.25) (layer "F.Cu") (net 8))
 (segment (start 134.35 98.8) (end 133.3 97.75) (width 0.25) (layer "F.Cu") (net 8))
 (segment (start 130 94) (end 128.5 94) (width 0.25) (layer "F.Cu") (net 8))
 (segment (start 128.5 94) (end 127.5 95) (width 0.25) (layer "F.Cu") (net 8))
 (segment (start 137.64 98.8) (end 137.39 98.8) (width 0.25) (layer "F.Cu") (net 8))
 (segment (start 133.3 97.75) (end 132.25 97.75) (width 0.25) (layer "F.Cu") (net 8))
 (segment (start 132.25 97.75) (end 131.25 96.75) (width 0.25) (layer "F.Cu") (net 8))
 (segment (start 140.1 101.26) (end 137.64 98.8) (width 0.25) (layer "F.Cu") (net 8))
 (segment (start 131.25 95.25) (end 130 94) (width 0.25) (layer "F.Cu") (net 8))
 (segment (start 139.89 106.34) (end 140.375 106.34) (width 0.254) (layer "F.Cu") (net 11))
 (segment (start 135.15 105.05) (end 138.6 105.05) (width 0.254) (layer "F.Cu") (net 11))
 (segment (start 138.6 105.05) (end 139.89 106.34) (width 0.254) (layer "F.Cu") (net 11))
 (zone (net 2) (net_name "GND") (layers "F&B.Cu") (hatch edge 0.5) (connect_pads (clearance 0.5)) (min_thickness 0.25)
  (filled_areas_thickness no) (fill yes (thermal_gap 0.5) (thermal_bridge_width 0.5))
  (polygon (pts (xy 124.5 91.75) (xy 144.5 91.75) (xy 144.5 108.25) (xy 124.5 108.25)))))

